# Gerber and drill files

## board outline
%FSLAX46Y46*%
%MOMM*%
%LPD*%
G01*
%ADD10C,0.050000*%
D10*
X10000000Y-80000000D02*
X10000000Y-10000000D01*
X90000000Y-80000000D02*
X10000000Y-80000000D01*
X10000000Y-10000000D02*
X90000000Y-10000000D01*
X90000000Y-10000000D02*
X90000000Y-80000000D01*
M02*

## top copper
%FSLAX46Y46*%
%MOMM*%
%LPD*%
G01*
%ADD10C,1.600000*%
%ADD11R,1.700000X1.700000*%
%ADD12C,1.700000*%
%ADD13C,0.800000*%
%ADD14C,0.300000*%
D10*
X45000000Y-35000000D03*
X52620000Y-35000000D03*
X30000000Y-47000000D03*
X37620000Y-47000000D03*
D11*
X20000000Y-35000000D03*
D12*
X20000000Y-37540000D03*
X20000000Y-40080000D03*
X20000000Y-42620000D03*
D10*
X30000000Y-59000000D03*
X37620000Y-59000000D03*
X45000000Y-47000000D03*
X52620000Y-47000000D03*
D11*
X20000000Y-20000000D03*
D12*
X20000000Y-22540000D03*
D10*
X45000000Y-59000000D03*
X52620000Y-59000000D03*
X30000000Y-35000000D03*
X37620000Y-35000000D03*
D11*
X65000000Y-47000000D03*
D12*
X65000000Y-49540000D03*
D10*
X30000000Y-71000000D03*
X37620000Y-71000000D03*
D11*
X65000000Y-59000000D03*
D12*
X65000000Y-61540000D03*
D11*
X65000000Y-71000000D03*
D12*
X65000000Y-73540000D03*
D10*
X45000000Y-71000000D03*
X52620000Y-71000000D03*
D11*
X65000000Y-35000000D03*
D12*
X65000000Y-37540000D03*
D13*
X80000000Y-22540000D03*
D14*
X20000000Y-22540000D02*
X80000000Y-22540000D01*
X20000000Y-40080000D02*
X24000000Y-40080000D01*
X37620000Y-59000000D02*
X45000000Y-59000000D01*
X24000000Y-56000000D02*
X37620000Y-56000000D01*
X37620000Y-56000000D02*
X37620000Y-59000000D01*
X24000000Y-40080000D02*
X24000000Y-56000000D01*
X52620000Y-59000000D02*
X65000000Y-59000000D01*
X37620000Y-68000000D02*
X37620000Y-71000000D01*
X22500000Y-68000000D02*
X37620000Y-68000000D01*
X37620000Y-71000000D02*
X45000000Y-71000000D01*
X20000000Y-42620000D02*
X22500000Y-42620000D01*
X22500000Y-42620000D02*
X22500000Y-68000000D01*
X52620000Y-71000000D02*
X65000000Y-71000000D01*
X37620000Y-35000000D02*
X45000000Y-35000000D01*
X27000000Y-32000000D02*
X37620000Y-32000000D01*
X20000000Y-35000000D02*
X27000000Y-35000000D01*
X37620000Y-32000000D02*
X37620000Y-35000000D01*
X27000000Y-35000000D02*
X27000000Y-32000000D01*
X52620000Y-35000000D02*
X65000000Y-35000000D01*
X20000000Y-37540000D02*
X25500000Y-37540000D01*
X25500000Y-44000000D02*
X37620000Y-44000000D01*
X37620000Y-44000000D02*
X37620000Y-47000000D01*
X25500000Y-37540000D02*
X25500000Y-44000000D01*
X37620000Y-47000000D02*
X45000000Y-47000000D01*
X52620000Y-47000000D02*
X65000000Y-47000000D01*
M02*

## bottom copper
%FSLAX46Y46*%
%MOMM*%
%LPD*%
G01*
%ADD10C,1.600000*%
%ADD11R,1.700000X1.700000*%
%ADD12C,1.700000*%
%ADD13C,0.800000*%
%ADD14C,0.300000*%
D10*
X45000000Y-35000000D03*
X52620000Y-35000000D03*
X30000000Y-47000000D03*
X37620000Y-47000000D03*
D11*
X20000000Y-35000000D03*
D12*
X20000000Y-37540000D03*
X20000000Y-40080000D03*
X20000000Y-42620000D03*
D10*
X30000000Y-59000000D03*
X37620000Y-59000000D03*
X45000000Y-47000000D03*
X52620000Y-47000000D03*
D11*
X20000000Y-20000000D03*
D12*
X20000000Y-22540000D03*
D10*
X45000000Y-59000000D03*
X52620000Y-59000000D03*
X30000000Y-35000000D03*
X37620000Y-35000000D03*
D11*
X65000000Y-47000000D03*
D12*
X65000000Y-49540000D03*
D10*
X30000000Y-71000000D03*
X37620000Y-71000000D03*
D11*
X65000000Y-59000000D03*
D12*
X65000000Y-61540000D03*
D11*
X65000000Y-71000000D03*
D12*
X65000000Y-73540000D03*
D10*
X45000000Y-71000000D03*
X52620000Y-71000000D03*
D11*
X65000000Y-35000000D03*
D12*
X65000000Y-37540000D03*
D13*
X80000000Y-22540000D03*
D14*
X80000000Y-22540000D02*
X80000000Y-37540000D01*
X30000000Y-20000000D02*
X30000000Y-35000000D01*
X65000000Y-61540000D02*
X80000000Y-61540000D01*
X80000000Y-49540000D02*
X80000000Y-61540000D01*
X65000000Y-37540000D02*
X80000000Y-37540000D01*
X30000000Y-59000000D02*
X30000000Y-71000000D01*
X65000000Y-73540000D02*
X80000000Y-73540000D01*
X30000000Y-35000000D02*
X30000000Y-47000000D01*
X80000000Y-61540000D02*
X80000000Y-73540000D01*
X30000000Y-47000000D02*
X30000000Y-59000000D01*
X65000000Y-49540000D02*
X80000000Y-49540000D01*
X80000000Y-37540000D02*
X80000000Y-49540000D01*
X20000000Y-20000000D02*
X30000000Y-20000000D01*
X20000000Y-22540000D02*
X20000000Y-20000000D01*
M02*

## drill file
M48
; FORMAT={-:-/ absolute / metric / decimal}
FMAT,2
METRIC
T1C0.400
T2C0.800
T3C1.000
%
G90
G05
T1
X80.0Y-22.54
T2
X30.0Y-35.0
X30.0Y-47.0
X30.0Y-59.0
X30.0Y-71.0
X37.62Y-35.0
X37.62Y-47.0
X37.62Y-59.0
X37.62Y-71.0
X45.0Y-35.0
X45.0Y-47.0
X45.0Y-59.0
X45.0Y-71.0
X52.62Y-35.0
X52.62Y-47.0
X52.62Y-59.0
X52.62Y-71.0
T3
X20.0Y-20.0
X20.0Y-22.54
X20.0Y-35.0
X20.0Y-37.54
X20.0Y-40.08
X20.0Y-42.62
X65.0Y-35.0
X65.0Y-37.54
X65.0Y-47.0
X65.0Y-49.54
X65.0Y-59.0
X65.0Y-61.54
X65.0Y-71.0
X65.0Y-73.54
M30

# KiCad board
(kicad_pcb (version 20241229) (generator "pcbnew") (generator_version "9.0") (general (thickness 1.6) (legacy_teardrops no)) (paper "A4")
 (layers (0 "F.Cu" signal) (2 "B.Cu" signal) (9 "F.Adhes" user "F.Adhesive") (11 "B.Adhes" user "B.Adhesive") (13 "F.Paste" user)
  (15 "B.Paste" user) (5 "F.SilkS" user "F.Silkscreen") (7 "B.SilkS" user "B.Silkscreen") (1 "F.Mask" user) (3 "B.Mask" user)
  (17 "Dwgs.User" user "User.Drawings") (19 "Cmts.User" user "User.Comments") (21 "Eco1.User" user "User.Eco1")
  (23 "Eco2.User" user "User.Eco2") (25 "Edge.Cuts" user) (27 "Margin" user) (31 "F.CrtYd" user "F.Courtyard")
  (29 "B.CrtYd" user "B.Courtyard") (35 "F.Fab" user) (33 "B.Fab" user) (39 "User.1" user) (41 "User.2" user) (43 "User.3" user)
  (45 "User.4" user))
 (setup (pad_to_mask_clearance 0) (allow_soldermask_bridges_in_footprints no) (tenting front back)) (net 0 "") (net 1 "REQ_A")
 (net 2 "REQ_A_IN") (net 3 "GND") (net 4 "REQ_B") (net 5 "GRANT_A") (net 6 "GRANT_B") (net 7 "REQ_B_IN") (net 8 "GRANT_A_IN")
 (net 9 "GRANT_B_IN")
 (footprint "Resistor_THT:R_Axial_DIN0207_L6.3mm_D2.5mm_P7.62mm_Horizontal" (layer "F.Cu") (at 45 35)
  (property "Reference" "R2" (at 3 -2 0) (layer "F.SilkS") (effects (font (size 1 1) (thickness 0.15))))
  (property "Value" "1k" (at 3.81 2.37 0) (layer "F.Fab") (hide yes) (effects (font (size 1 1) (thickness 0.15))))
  (pad "1" thru_hole circle (at 0 0) (size 1.6 1.6) (drill 0.8) (layers "*.Cu" "*.Mask") (remove_unused_layers no) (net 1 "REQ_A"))
  (pad "2" thru_hole circle (at 7.62 0) (size 1.6 1.6) (drill 0.8) (layers "*.Cu" "*.Mask") (remove_unused_layers no) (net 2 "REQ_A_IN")))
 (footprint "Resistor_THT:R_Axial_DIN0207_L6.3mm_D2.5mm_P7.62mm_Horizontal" (layer "F.Cu") (at 30 47)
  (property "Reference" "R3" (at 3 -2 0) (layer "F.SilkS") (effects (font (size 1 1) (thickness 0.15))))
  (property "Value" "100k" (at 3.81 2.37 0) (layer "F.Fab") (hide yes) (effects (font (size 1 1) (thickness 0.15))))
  (pad "1" thru_hole circle (at 0 0) (size 1.6 1.6) (drill 0.8) (layers "*.Cu" "*.Mask") (remove_unused_layers no) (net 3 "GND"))
  (pad "2" thru_hole circle (at 7.62 0) (size 1.6 1.6) (drill 0.8) (layers "*.Cu" "*.Mask") (remove_unused_layers no) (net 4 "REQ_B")))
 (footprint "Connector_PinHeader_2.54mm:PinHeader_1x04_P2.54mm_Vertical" (layer "F.Cu") (at 20 35)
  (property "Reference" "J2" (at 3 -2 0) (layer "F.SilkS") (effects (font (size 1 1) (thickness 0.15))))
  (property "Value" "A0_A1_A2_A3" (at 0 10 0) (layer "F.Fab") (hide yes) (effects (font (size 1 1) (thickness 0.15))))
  (pad "1" thru_hole rect (at 0 0) (size 1.7 1.7) (drill 1) (layers "*.Cu" "*.Mask") (remove_unused_layers no) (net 1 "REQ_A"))
  (pad "2" thru_hole circle (at 0 2.54) (size 1.7 1.7) (drill 1) (layers "*.Cu" "*.Mask") (remove_unused_layers no) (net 4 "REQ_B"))
  (pad "3" thru_hole circle (at 0 5.08) (size 1.7 1.7) (drill 1) (layers "*.Cu" "*.Mask") (remove_unused_layers no) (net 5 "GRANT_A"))
  (pad "4" thru_hole circle (at 0 7.62) (size 1.7 1.7) (drill 1) (layers "*.Cu" "*.Mask") (remove_unused_layers no) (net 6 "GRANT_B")))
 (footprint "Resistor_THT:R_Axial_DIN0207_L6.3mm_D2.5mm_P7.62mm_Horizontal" (layer "F.Cu") (at 30 59)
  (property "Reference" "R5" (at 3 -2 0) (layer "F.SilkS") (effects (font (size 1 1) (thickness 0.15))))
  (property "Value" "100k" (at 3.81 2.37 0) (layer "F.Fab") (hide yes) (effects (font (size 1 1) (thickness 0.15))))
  (pad "1" thru_hole circle (at 0 0) (size 1.6 1.6) (drill 0.8) (layers "*.Cu" "*.Mask") (remove_unused_layers no) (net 3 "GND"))
  (pad "2" thru_hole circle (at 7.62 0) (size 1.6 1.6) (drill 0.8) (layers "*.Cu" "*.Mask") (remove_unused_layers no) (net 5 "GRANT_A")))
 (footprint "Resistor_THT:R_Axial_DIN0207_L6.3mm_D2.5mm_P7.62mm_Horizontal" (layer "F.Cu") (at 45 47)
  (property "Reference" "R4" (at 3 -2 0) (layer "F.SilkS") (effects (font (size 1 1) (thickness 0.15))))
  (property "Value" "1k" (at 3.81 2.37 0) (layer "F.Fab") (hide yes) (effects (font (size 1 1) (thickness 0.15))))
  (pad "1" thru_hole circle (at 0 0) (size 1.6 1.6) (drill 0.8) (layers "*.Cu" "*.Mask") (remove_unused_layers no) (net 4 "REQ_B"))
  (pad "2" thru_hole circle (at 7.62 0) (size 1.6 1.6) (drill 0.8) (layers "*.Cu" "*.Mask") (remove_unused_layers no) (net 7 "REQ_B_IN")))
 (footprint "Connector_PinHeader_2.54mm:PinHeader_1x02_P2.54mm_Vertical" (layer "F.Cu") (at 20 20)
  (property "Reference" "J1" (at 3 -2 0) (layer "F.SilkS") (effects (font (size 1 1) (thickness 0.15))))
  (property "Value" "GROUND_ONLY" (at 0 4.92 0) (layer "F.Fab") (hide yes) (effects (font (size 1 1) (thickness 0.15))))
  (pad "1" thru_hole rect (at 0 0) (size 1.7 1.7) (drill 1) (layers "*.Cu" "*.Mask") (remove_unused_layers no) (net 3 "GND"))
  (pad "2" thru_hole circle (at 0 2.54) (size 1.7 1.7) (drill 1) (layers "*.Cu" "*.Mask") (remove_unused_layers no) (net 3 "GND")))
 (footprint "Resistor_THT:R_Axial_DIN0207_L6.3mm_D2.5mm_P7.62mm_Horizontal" (layer "F.Cu") (at 45 59)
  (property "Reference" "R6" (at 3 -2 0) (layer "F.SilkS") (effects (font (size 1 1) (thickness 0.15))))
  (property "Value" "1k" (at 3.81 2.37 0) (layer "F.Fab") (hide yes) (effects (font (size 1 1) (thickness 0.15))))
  (pad "1" thru_hole circle (at 0 0) (size 1.6 1.6) (drill 0.8) (layers "*.Cu" "*.Mask") (remove_unused_layers no) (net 5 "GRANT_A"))
  (pad "2" thru_hole circle (at 7.62 0) (size 1.6 1.6) (drill 0.8) (layers "*.Cu" "*.Mask") (remove_unused_layers no) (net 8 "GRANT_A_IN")))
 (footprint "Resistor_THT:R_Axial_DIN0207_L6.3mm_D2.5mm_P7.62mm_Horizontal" (layer "F.Cu") (at 30 35)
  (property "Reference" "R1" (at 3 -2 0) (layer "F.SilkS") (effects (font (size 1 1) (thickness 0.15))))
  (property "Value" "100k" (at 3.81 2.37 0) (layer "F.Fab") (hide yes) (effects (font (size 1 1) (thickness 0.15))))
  (pad "1" thru_hole circle (at 0 0) (size 1.6 1.6) (drill 0.8) (layers "*.Cu" "*.Mask") (remove_unused_layers no) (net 3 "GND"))
  (pad "2" thru_hole circle (at 7.62 0) (size 1.6 1.6) (drill 0.8) (layers "*.Cu" "*.Mask") (remove_unused_layers no) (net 1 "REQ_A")))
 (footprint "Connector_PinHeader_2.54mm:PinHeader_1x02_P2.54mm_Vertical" (layer "F.Cu") (at 65 47)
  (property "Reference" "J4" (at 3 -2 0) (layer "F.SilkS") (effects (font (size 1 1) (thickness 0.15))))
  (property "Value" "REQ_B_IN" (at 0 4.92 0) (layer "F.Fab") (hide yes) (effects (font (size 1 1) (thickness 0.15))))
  (pad "1" thru_hole rect (at 0 0) (size 1.7 1.7) (drill 1) (layers "*.Cu" "*.Mask") (remove_unused_layers no) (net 7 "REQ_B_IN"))
  (pad "2" thru_hole circle (at 0 2.54) (size 1.7 1.7) (drill 1) (layers "*.Cu" "*.Mask") (remove_unused_layers no) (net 3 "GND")))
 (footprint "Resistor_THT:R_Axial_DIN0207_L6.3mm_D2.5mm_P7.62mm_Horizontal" (layer "F.Cu") (at 30 71)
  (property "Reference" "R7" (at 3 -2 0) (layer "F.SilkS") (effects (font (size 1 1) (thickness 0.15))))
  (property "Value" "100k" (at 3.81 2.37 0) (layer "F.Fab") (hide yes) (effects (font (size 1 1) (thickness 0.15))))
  (pad "1" thru_hole circle (at 0 0) (size 1.6 1.6) (drill 0.8) (layers "*.Cu" "*.Mask") (remove_unused_layers no) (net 3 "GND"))
  (pad "2" thru_hole circle (at 7.62 0) (size 1.6 1.6) (drill 0.8) (layers "*.Cu" "*.Mask") (remove_unused_layers no) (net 6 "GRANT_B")))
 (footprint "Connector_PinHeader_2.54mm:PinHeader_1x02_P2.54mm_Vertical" (layer "F.Cu") (at 65 59)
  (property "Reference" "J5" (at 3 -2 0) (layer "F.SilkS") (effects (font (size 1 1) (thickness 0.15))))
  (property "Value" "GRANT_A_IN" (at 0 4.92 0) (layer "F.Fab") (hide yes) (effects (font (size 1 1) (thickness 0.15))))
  (pad "1" thru_hole rect (at 0 0) (size 1.7 1.7) (drill 1) (layers "*.Cu" "*.Mask") (remove_unused_layers no) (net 8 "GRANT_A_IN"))
  (pad "2" thru_hole circle (at 0 2.54) (size 1.7 1.7) (drill 1) (layers "*.Cu" "*.Mask") (remove_unused_layers no) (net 3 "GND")))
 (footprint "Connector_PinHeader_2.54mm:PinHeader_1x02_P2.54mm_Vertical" (layer "F.Cu") (at 65 71)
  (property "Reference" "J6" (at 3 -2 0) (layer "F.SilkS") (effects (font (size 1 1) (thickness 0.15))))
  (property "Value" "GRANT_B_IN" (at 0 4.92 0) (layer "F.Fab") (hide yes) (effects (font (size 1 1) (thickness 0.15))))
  (pad "1" thru_hole rect (at 0 0) (size 1.7 1.7) (drill 1) (layers "*.Cu" "*.Mask") (remove_unused_layers no) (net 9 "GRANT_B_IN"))
  (pad "2" thru_hole circle (at 0 2.54) (size 1.7 1.7) (drill 1) (layers "*.Cu" "*.Mask") (remove_unused_layers no) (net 3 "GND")))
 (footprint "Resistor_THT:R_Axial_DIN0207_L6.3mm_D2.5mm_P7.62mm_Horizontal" (layer "F.Cu") (at 45 71)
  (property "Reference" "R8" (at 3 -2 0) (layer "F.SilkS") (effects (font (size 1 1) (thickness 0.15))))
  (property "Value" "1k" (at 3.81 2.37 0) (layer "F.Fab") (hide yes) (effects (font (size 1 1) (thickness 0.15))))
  (pad "1" thru_hole circle (at 0 0) (size 1.6 1.6) (drill 0.8) (layers "*.Cu" "*.Mask") (remove_unused_layers no) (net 6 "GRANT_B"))
  (pad "2" thru_hole circle (at 7.62 0) (size 1.6 1.6) (drill 0.8) (layers "*.Cu" "*.Mask") (remove_unused_layers no) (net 9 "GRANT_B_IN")))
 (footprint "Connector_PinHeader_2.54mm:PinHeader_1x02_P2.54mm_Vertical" (layer "F.Cu") (at 65 35)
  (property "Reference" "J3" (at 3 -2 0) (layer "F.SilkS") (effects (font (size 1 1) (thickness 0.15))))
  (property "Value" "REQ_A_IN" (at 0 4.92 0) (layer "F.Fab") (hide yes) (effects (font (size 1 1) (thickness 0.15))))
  (pad "1" thru_hole rect (at 0 0) (size 1.7 1.7) (drill 1) (layers "*.Cu" "*.Mask") (remove_unused_layers no) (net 2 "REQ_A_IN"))
  (pad "2" thru_hole circle (at 0 2.54) (size 1.7 1.7) (drill 1) (layers "*.Cu" "*.Mask") (remove_unused_layers no) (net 3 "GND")))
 (gr_line (start 10 80) (end 10 10) (stroke (width 0.05) (type default)) (layer "Edge.Cuts"))
 (gr_line (start 90 80) (end 10 80) (stroke (width 0.05) (type default)) (layer "Edge.Cuts"))
 (gr_line (start 10 10) (end 90 10) (stroke (width 0.05) (type default)) (layer "Edge.Cuts"))
 (gr_line (start 90 10) (end 90 80) (stroke (width 0.05) (type default)) (layer "Edge.Cuts"))
 (segment (start 20 22.54) (end 80 22.54) (width 0.3) (layer "F.Cu") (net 3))
 (via (at 80 22.54) (size 0.8) (drill 0.4) (layers "F.Cu" "B.Cu") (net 3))
 (segment (start 80 22.54) (end 80 37.54) (width 0.3) (layer "B.Cu") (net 3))
 (segment (start 30 20) (end 30 35) (width 0.3) (layer "B.Cu") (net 3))
 (segment (start 65 61.54) (end 80 61.54) (width 0.3) (layer "B.Cu") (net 3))
 (segment (start 80 49.54) (end 80 61.54) (width 0.3) (layer "B.Cu") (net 3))
 (segment (start 65 37.54) (end 80 37.54) (width 0.3) (layer "B.Cu") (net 3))
 (segment (start 30 59) (end 30 71) (width 0.3) (layer "B.Cu") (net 3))
 (segment (start 65 73.54) (end 80 73.54) (width 0.3) (layer "B.Cu") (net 3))
 (segment (start 30 35) (end 30 47) (width 0.3) (layer "B.Cu") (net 3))
 (segment (start 80 61.54) (end 80 73.54) (width 0.3) (layer "B.Cu") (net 3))
 (segment (start 30 47) (end 30 59) (width 0.3) (layer "B.Cu") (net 3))
 (segment (start 65 49.54) (end 80 49.54) (width 0.3) (layer "B.Cu") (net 3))
 (segment (start 80 37.54) (end 80 49.54) (width 0.3) (layer "B.Cu") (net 3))
 (segment (start 20 20) (end 30 20) (width 0.3) (layer "B.Cu") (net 3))
 (segment (start 20 22.54) (end 20 20) (width 0.3) (layer "B.Cu") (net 3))
 (segment (start 20 40.08) (end 24 40.08) (width 0.3) (layer "F.Cu") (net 5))
 (segment (start 37.62 59) (end 45 59) (width 0.3) (layer "F.Cu") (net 5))
 (segment (start 24 56) (end 37.62 56) (width 0.3) (layer "F.Cu") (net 5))
 (segment (start 37.62 56) (end 37.62 59) (width 0.3) (layer "F.Cu") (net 5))
 (segment (start 24 40.08) (end 24 56) (width 0.3) (layer "F.Cu") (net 5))
 (segment (start 52.62 59) (end 65 59) (width 0.3) (layer "F.Cu") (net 8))
 (segment (start 37.62 68) (end 37.62 71) (width 0.3) (layer "F.Cu") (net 6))
 (segment (start 22.5 68) (end 37.62 68) (width 0.3) (layer "F.Cu") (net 6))
 (segment (start 37.62 71) (end 45 71) (width 0.3) (layer "F.Cu") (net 6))
 (segment (start 20 42.62) (end 22.5 42.62) (width 0.3) (layer "F.Cu") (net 6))
 (segment (start 22.5 42.62) (end 22.5 68) (width 0.3) (layer "F.Cu") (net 6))
 (segment (start 52.62 71) (end 65 71) (width 0.3) (layer "F.Cu") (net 9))
 (segment (start 37.62 35) (end 45 35) (width 0.3) (layer "F.Cu") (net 1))
 (segment (start 27 32) (end 37.62 32) (width 0.3) (layer "F.Cu") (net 1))
 (segment (start 20 35) (end 27 35) (width 0.3) (layer "F.Cu") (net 1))
 (segment (start 37.62 32) (end 37.62 35) (width 0.3) (layer "F.Cu") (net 1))
 (segment (start 27 35) (end 27 32) (width 0.3) (layer "F.Cu") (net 1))
 (segment (start 52.62 35) (end 65 35) (width 0.3) (layer "F.Cu") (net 2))
 (segment (start 20 37.54) (end 25.5 37.54) (width 0.3) (layer "F.Cu") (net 4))
 (segment (start 25.5 44) (end 37.62 44) (width 0.3) (layer "F.Cu") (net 4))
 (segment (start 37.62 44) (end 37.62 47) (width 0.3) (layer "F.Cu") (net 4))
 (segment (start 25.5 37.54) (end 25.5 44) (width 0.3) (layer "F.Cu") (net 4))
 (segment (start 37.62 47) (end 45 47) (width 0.3) (layer "F.Cu") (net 4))
 (segment (start 52.62 47) (end 65 47) (width 0.3) (layer "F.Cu") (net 7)))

